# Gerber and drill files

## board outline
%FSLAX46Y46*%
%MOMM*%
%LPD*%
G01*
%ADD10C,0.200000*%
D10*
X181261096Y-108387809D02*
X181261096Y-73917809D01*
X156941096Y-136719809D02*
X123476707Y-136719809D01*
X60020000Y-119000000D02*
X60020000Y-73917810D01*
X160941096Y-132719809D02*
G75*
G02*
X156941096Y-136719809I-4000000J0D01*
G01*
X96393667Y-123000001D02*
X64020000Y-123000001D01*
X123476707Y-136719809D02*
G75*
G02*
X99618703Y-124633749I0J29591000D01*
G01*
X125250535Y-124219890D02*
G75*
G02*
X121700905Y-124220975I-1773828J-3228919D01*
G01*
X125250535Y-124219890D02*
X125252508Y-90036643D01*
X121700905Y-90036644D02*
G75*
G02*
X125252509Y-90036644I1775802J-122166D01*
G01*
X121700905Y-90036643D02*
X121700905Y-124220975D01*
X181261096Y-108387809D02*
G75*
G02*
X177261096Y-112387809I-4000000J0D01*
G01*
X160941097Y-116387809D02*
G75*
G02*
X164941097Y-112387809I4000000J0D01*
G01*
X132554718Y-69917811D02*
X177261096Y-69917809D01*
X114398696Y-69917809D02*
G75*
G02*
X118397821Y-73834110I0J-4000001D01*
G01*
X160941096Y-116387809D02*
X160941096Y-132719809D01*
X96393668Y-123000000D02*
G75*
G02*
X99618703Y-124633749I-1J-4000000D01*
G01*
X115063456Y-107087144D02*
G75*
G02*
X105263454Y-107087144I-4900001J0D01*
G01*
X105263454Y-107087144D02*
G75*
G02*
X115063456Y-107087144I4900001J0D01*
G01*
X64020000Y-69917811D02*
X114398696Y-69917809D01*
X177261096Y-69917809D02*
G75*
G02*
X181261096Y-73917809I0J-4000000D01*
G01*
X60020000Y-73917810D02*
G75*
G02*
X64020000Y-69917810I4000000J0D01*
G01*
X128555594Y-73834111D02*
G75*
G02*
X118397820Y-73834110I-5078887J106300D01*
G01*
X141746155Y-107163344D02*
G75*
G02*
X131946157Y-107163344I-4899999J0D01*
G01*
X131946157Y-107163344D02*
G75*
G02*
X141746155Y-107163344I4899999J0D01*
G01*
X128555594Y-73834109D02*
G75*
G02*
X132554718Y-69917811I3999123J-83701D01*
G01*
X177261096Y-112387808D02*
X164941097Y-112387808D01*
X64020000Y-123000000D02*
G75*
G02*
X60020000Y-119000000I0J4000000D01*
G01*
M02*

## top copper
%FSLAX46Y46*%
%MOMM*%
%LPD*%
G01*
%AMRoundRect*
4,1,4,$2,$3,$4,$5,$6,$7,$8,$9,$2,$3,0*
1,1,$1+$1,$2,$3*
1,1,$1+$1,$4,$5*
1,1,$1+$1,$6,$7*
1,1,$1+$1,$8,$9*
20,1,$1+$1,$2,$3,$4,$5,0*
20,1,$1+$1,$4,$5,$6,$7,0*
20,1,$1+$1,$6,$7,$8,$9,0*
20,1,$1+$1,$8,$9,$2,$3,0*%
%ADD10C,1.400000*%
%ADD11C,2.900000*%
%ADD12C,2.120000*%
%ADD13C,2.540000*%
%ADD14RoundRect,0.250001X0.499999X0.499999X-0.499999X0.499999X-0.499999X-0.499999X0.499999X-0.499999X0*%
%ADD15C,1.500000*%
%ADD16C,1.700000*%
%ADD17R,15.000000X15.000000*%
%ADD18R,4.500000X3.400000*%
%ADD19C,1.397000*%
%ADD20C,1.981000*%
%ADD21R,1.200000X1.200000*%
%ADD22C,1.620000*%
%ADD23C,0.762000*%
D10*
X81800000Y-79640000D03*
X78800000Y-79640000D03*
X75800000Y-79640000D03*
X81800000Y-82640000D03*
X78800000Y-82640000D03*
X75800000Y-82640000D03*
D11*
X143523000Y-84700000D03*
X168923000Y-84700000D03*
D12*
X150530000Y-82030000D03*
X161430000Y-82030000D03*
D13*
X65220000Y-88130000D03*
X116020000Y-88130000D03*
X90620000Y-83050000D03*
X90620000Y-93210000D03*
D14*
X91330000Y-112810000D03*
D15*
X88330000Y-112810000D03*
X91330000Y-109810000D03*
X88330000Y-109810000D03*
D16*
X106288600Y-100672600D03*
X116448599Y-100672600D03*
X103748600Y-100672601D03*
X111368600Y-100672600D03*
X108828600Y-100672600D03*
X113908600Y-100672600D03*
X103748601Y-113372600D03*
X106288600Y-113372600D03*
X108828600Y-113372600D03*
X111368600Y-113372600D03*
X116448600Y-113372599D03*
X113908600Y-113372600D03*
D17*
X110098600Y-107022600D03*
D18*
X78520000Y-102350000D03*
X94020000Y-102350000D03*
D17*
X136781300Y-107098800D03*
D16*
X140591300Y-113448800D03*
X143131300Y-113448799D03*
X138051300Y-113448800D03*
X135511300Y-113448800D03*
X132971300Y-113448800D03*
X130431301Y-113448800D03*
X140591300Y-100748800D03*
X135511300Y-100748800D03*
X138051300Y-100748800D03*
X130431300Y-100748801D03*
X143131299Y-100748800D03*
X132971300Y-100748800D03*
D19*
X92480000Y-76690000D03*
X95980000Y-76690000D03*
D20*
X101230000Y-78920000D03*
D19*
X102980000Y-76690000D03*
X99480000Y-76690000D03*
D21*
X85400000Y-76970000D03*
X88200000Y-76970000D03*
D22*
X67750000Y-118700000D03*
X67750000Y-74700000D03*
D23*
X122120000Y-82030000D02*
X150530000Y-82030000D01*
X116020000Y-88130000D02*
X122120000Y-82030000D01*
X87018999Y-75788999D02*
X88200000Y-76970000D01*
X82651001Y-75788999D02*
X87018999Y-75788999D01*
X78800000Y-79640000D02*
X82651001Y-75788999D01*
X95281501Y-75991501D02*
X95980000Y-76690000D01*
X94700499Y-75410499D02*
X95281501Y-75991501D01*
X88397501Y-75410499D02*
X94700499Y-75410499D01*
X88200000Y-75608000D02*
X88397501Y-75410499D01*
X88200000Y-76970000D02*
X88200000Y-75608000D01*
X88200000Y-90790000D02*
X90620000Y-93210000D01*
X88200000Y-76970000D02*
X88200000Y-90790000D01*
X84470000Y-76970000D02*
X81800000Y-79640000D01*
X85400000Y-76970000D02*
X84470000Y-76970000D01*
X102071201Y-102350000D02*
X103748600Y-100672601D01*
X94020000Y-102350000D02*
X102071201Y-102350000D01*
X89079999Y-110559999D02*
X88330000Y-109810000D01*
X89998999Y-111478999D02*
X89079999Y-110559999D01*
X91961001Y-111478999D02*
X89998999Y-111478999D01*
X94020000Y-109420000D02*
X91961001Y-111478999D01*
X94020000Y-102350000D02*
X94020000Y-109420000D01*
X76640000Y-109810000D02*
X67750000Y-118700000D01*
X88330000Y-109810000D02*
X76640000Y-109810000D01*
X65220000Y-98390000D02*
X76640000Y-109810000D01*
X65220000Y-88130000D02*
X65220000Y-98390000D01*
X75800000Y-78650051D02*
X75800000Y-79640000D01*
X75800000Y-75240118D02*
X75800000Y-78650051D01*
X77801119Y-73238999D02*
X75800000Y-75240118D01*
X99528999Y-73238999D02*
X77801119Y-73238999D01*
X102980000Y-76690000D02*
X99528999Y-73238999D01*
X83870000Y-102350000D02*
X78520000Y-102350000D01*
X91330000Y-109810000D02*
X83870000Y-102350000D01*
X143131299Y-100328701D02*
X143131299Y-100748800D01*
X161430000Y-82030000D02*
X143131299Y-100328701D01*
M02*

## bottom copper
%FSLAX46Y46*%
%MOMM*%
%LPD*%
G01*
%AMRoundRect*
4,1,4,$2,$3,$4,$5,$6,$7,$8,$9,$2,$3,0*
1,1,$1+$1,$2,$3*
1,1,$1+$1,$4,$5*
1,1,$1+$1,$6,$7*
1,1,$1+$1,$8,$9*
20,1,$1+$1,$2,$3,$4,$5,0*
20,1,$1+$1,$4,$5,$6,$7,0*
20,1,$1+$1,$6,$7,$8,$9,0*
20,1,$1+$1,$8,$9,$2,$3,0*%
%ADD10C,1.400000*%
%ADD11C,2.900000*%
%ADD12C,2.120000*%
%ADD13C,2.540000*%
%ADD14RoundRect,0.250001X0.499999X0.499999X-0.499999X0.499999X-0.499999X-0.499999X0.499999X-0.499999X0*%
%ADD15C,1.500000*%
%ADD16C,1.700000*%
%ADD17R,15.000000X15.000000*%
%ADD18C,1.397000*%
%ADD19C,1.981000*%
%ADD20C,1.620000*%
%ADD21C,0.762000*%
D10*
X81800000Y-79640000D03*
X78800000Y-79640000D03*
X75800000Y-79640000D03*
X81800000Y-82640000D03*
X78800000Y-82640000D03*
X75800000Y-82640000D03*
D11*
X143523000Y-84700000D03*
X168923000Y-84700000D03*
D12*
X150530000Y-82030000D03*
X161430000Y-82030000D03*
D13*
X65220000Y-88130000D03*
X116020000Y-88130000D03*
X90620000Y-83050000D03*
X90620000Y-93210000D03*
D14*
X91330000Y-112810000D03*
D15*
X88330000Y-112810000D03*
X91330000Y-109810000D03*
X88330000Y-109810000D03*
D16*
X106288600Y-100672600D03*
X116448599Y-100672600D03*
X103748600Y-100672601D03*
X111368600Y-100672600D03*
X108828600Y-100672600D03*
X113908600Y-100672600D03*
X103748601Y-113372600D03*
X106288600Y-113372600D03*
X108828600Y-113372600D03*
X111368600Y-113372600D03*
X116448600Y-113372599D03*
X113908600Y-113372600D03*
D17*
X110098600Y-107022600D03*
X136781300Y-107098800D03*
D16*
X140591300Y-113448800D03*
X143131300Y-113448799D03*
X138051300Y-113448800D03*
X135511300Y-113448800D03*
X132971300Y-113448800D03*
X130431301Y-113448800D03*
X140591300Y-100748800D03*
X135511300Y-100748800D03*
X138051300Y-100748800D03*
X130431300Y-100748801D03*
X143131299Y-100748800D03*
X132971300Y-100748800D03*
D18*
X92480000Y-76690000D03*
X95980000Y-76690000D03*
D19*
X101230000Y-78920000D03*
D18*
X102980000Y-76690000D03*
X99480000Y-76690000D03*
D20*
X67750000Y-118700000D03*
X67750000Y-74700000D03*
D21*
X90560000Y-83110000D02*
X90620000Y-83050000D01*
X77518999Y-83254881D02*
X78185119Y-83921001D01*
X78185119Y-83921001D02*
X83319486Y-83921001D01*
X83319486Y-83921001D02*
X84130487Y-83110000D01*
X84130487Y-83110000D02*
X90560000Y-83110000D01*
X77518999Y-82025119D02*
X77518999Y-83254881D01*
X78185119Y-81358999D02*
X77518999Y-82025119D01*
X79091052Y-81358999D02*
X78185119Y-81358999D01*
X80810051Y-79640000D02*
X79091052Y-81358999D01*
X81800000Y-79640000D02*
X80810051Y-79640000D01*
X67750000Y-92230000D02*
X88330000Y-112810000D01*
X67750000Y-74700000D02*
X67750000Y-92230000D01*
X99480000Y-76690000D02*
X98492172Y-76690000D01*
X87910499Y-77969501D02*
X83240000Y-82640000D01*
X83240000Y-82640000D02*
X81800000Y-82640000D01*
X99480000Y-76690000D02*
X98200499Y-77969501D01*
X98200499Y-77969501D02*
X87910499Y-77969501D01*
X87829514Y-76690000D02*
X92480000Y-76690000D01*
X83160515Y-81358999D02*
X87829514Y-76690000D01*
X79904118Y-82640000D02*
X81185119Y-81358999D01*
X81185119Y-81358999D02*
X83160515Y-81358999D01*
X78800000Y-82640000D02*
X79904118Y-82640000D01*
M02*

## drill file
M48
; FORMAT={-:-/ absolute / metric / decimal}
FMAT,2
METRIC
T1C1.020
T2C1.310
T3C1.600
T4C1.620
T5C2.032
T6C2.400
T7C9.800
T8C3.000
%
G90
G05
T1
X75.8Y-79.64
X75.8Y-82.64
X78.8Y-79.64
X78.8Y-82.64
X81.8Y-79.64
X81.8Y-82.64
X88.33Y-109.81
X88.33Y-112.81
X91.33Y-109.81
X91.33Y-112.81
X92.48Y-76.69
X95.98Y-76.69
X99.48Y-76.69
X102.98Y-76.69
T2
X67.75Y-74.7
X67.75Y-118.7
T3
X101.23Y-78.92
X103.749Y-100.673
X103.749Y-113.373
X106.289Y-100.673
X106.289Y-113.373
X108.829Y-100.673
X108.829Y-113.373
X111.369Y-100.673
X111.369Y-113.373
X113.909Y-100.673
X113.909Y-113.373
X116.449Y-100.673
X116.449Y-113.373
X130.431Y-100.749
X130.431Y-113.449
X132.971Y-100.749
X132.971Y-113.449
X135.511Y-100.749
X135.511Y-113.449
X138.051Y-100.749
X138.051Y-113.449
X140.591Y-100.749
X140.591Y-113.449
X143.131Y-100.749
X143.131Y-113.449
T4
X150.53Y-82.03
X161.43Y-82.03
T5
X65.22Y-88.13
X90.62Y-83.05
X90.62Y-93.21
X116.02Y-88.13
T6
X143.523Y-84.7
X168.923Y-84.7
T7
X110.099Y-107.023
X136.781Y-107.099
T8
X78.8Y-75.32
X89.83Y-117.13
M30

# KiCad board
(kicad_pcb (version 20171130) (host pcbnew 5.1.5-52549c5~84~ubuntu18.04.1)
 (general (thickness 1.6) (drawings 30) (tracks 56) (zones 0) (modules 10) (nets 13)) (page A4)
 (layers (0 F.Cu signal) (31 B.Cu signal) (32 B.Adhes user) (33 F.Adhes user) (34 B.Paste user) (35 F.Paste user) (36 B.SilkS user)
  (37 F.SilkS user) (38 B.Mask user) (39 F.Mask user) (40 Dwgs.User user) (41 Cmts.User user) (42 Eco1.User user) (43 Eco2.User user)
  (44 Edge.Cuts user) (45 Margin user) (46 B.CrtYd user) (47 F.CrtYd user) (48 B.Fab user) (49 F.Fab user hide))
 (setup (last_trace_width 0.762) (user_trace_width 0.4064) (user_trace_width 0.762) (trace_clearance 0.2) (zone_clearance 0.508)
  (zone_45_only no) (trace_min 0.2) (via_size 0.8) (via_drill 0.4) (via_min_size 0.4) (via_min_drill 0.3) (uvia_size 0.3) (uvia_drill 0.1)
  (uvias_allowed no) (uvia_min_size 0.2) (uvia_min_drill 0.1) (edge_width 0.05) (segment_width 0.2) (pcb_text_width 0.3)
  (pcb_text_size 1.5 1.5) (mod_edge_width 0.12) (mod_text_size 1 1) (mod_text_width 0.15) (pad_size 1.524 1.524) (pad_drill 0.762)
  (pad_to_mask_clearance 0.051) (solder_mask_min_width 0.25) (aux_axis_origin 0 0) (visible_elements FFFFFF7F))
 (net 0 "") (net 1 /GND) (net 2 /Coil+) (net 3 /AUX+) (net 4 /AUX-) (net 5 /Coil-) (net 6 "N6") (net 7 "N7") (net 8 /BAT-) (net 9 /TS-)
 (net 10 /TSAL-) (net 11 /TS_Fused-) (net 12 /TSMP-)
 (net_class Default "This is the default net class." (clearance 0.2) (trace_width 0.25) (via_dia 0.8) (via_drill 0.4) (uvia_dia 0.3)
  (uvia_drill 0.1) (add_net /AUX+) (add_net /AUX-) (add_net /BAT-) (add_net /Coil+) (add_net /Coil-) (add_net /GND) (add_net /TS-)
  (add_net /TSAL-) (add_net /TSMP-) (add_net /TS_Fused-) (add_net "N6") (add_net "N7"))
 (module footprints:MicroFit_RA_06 (layer B.Cu) (at 78.8 75.32 180)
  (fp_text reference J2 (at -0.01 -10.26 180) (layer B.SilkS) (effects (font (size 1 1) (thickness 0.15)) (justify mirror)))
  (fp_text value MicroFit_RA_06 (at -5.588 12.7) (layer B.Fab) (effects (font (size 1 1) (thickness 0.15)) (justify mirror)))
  (pad "" np_thru_hole circle (at 0 0) (size 3 3) (drill 3) (layers *.Cu *.Mask))
  (pad 1 thru_hole circle (at -3 -4.32) (size 1.4 1.4) (drill 1.02) (layers *.Cu *.Mask) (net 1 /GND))
  (pad 2 thru_hole circle (at 0 -4.32) (size 1.4 1.4) (drill 1.02) (layers *.Cu *.Mask) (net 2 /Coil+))
  (pad 3 thru_hole circle (at 3 -4.32) (size 1.4 1.4) (drill 1.02) (layers *.Cu *.Mask) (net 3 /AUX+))
  (pad 4 thru_hole circle (at -3 -7.32) (size 1.4 1.4) (drill 1.02) (layers *.Cu *.Mask) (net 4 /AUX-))
  (pad 5 thru_hole circle (at 0 -7.32) (size 1.4 1.4) (drill 1.02) (layers *.Cu *.Mask) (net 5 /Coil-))
  (pad 6 thru_hole circle (at 3 -7.32) (size 1.4 1.4) (drill 1.02) (layers *.Cu *.Mask) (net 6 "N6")))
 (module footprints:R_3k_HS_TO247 (layer F.Cu) (at 161.43 82.03 180)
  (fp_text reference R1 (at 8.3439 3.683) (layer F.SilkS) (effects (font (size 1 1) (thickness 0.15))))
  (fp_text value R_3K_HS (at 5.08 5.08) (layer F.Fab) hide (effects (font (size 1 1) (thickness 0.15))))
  (pad 5 thru_hole circle (at 17.907 -2.67 180) (size 2.9 2.9) (drill 2.4) (layers *.Cu *.Mask))
  (pad 4 thru_hole circle (at -7.493 -2.67 180) (size 2.9 2.9) (drill 2.4) (layers *.Cu *.Mask))
  (pad 2 thru_hole circle (at 10.9 0 180) (size 2.12 2.12) (drill 1.62) (layers *.Cu *.Mask) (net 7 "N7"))
  (pad 1 thru_hole circle (at 0 0 180) (size 2.12 2.12) (drill 1.62) (layers *.Cu *.Mask) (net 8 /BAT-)))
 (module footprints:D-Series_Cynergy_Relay (layer F.Cu) (at 65.22 88.13)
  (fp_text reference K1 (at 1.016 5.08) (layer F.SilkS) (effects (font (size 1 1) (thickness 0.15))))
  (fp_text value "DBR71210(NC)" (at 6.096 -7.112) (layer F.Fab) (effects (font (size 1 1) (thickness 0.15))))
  (pad 1 thru_hole circle (at 0 0) (size 2.54 2.54) (drill 2.032) (layers *.Cu *.Mask) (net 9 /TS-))
  (pad 2 thru_hole circle (at 50.8 0) (size 2.54 2.54) (drill 2.032) (layers *.Cu *.Mask) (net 7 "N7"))
  (pad 3 thru_hole circle (at 25.4 -5.08) (size 2.54 2.54) (drill 2.032) (layers *.Cu *.Mask) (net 1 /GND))
  (pad 4 thru_hole circle (at 25.4 5.08) (size 2.54 2.54) (drill 2.032) (layers *.Cu *.Mask) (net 2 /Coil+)))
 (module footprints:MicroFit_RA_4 (layer F.Cu) (at 91.33 112.81 180)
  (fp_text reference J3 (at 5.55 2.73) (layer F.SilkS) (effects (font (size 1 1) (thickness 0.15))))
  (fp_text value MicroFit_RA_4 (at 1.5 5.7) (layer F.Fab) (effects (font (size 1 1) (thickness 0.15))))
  (pad "" np_thru_hole circle (at 1.5 -4.32 180) (size 3 3) (drill 3) (layers *.Cu *.Mask))
  (pad 1 thru_hole roundrect (at 0 0 180) (size 1.5 1.5) (drill 1.02) (layers *.Cu *.Mask) (roundrect_rratio 0.166667) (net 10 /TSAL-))
  (pad 2 thru_hole circle (at 3 0 180) (size 1.5 1.5) (drill 1.02) (layers *.Cu *.Mask) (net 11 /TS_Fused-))
  (pad 3 thru_hole circle (at 0 3 180) (size 1.5 1.5) (drill 1.02) (layers *.Cu *.Mask) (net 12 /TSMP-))
  (pad 4 thru_hole circle (at 3 3 180) (size 1.5 1.5) (drill 1.02) (layers *.Cu *.Mask) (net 9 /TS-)))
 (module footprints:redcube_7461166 (layer F.Cu) (at 110.0986 107.0226)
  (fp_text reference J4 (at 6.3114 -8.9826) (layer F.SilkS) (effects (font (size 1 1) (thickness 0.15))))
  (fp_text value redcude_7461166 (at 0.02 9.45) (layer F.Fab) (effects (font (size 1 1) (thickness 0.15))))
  (pad 1 thru_hole circle (at -3.81 -6.35) (size 1.7 1.7) (drill 1.6) (layers *.Cu *.Mask) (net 9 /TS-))
  (pad 1 thru_hole circle (at 6.349999 -6.35) (size 1.7 1.7) (drill 1.6) (layers *.Cu *.Mask) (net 9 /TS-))
  (pad 1 thru_hole circle (at -6.35 -6.349999) (size 1.7 1.7) (drill 1.6) (layers *.Cu *.Mask) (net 9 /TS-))
  (pad 1 thru_hole circle (at 1.27 -6.35) (size 1.7 1.7) (drill 1.6) (layers *.Cu *.Mask) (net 9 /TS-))
  (pad 1 thru_hole circle (at -1.27 -6.35) (size 1.7 1.7) (drill 1.6) (layers *.Cu *.Mask) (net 9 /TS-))
  (pad 1 thru_hole circle (at 3.81 -6.35) (size 1.7 1.7) (drill 1.6) (layers *.Cu *.Mask) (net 9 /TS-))
  (pad 1 thru_hole circle (at -6.349999 6.35) (size 1.7 1.7) (drill 1.6) (layers *.Cu *.Mask) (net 9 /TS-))
  (pad 1 thru_hole circle (at -3.81 6.35) (size 1.7 1.7) (drill 1.6) (layers *.Cu *.Mask) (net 9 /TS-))
  (pad 1 thru_hole circle (at -1.27 6.35) (size 1.7 1.7) (drill 1.6) (layers *.Cu *.Mask) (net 9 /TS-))
  (pad 1 thru_hole circle (at 1.27 6.35) (size 1.7 1.7) (drill 1.6) (layers *.Cu *.Mask) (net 9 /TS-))
  (pad 1 thru_hole circle (at 6.35 6.349999) (size 1.7 1.7) (drill 1.6) (layers *.Cu *.Mask) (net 9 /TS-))
  (pad 1 thru_hole circle (at 3.81 6.35) (size 1.7 1.7) (drill 1.6) (layers *.Cu *.Mask) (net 9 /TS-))
  (pad 1 thru_hole rect (at 0 0) (size 15 15) (drill 9.8) (layers *.Cu *.Mask) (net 9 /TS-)))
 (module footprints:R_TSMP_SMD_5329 (layer F.Cu) (at 86.14 102.35)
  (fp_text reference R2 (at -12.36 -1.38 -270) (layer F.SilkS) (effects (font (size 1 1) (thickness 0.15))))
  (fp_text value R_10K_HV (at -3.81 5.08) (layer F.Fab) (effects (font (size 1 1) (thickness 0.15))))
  (pad 1 smd rect (at -7.62 0) (size 4.5 3.4) (layers F.Cu F.Paste F.Mask) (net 12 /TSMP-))
  (pad 2 smd rect (at 7.88 0) (size 4.5 3.4) (layers F.Cu F.Paste F.Mask) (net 9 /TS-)))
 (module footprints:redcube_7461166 (layer F.Cu) (at 136.7813 107.0988)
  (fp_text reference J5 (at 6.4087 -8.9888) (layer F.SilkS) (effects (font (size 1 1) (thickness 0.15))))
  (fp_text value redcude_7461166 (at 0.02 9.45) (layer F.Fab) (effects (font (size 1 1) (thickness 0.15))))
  (pad 1 thru_hole rect (at 0 0) (size 15 15) (drill 9.8) (layers *.Cu *.Mask) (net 8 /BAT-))
  (pad 1 thru_hole circle (at 3.81 6.35) (size 1.7 1.7) (drill 1.6) (layers *.Cu *.Mask) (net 8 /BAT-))
  (pad 1 thru_hole circle (at 6.35 6.349999) (size 1.7 1.7) (drill 1.6) (layers *.Cu *.Mask) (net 8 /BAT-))
  (pad 1 thru_hole circle (at 1.27 6.35) (size 1.7 1.7) (drill 1.6) (layers *.Cu *.Mask) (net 8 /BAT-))
  (pad 1 thru_hole circle (at -1.27 6.35) (size 1.7 1.7) (drill 1.6) (layers *.Cu *.Mask) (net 8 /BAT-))
  (pad 1 thru_hole circle (at -3.81 6.35) (size 1.7 1.7) (drill 1.6) (layers *.Cu *.Mask) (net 8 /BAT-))
  (pad 1 thru_hole circle (at -6.349999 6.35) (size 1.7 1.7) (drill 1.6) (layers *.Cu *.Mask) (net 8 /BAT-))
  (pad 1 thru_hole circle (at 3.81 -6.35) (size 1.7 1.7) (drill 1.6) (layers *.Cu *.Mask) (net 8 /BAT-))
  (pad 1 thru_hole circle (at -1.27 -6.35) (size 1.7 1.7) (drill 1.6) (layers *.Cu *.Mask) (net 8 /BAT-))
  (pad 1 thru_hole circle (at 1.27 -6.35) (size 1.7 1.7) (drill 1.6) (layers *.Cu *.Mask) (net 8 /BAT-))
  (pad 1 thru_hole circle (at -6.35 -6.349999) (size 1.7 1.7) (drill 1.6) (layers *.Cu *.Mask) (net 8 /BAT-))
  (pad 1 thru_hole circle (at 6.349999 -6.35) (size 1.7 1.7) (drill 1.6) (layers *.Cu *.Mask) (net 8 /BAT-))
  (pad 1 thru_hole circle (at -3.81 -6.35) (size 1.7 1.7) (drill 1.6) (layers *.Cu *.Mask) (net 8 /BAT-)))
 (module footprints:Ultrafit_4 (layer B.Cu) (at 97.73 76.69 270)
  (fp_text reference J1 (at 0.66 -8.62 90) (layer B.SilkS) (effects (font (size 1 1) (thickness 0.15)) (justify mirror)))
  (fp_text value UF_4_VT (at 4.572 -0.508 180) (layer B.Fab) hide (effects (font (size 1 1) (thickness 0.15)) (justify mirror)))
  (pad 4 thru_hole circle (at 0 5.25 90) (size 1.397 1.397) (drill 1.02) (layers *.Cu *.Mask) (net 5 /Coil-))
  (pad 3 thru_hole circle (at 0 1.75 90) (size 1.397 1.397) (drill 1.02) (layers *.Cu *.Mask) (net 2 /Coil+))
  (pad "" thru_hole circle (at 2.23 -3.5 270) (size 1.981 1.981) (drill 1.6) (layers *.Cu *.Mask))
  (pad 1 thru_hole circle (at 0 -5.25 270) (size 1.397 1.397) (drill 1.02) (layers *.Cu *.Mask) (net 3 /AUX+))
  (pad 2 thru_hole circle (at 0 -1.75 270) (size 1.397 1.397) (drill 1.02) (layers *.Cu *.Mask) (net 4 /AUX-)))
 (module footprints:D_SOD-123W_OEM (layer F.Cu) (at 86.8 76.97 180)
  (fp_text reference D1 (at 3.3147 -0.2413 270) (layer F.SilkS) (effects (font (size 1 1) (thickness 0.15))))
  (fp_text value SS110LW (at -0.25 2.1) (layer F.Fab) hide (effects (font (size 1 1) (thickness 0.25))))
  (pad 2 smd rect (at 1.4 0 180) (size 1.2 1.2) (layers F.Cu F.Paste F.Mask) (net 1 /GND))
  (pad 1 smd rect (at -1.4 0 180) (size 1.2 1.2) (layers F.Cu F.Paste F.Mask) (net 2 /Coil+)))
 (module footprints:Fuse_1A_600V (layer B.Cu) (at 67.75 118.7 90)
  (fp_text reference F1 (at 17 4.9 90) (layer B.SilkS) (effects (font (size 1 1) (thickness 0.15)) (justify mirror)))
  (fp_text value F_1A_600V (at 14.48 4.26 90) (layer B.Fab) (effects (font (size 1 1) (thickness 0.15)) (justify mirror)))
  (pad 1 thru_hole circle (at 0 0 90) (size 1.62 1.62) (drill 1.31) (layers *.Cu *.Mask) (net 9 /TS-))
  (pad 2 thru_hole circle (at 44 0 90) (size 1.62 1.62) (drill 1.31) (layers *.Cu *.Mask) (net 11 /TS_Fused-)))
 (gr_line (start 181.261096 108.387809) (end 181.261096 73.917809) (layer Edge.Cuts) (width 0.2))
 (gr_line (start 156.941096 136.719809) (end 123.476707 136.719809) (layer Edge.Cuts) (width 0.2))
 (gr_line (start 60.02 119) (end 60.02 73.91781) (layer Edge.Cuts) (width 0.2))
 (gr_arc (start 156.941096 132.719809) (end 156.941096 136.719809) (angle -90) (layer Edge.Cuts) (width 0.2))
 (gr_line (start 96.393667 123.000001) (end 64.02 123.000001) (layer Edge.Cuts) (width 0.2))
 (gr_arc (start 123.476707 107.128809) (end 99.618703 124.633749) (angle -53.73199979) (layer Edge.Cuts) (width 0.2))
 (gr_arc (start 123.476707 127.448809) (end 121.700905 124.220975) (angle -302.4) (layer Edge.Cuts) (width 0.2))
 (gr_line (start 125.250535 124.21989) (end 125.252508 90.036643) (layer Edge.Cuts) (width 0.2))
 (gr_arc (start 123.476707 90.15881) (end 125.252509 90.036644) (angle -172.1290943) (layer Edge.Cuts) (width 0.2))
 (gr_line (start 121.700905 90.036643) (end 121.700905 124.220975) (layer Edge.Cuts) (width 0.2))
 (gr_arc (start 177.261096 108.387809) (end 177.261096 112.387809) (angle -90) (layer Edge.Cuts) (width 0.2))
 (gr_arc (start 164.941097 116.387809) (end 164.941097 112.387809) (angle -90) (layer Edge.Cuts) (width 0.2))
 (gr_line (start 132.554718 69.917811) (end 177.261096 69.917809) (layer Edge.Cuts) (width 0.2))
 (gr_arc (start 114.398696 73.91781) (end 118.397821 73.83411) (angle -88.80099199) (layer Edge.Cuts) (width 0.2))
 (gr_line (start 160.941096 116.387809) (end 160.941096 132.719809) (layer Edge.Cuts) (width 0.2))
 (gr_arc (start 96.393667 127) (end 99.618703 124.633749) (angle -53.73200771) (layer Edge.Cuts) (width 0.2))
 (gr_circle (center 110.163455 107.087144) (end 115.063456 107.087144) (layer Edge.Cuts) (width 0.2))
 (gr_line (start 64.02 69.917811) (end 114.398696 69.917809) (layer Edge.Cuts) (width 0.2))
 (gr_arc (start 177.261096 73.917809) (end 181.261096 73.917809) (angle -90.00000194) (layer Edge.Cuts) (width 0.2))
 (gr_arc (start 64.02 73.91781) (end 64.02 69.91781) (angle -90) (layer Edge.Cuts) (width 0.2))
 (gr_arc (start 123.476707 73.727811) (end 118.39782 73.83411) (angle -177.6019899) (layer Edge.Cuts) (width 0.2))
 (gr_circle (center 136.846156 107.163344) (end 141.746155 107.163344) (layer Edge.Cuts) (width 0.2))
 (gr_arc (start 132.554717 73.91781) (end 132.554718 69.917811) (angle -88.80099199) (layer Edge.Cuts) (width 0.2))
 (gr_line (start 177.261096 112.387808) (end 164.941097 112.387808) (layer Edge.Cuts) (width 0.2))
 (gr_arc (start 64.02 119) (end 60.02 119) (angle -90) (layer Edge.Cuts) (width 0.2))
 (segment (start 122.12 82.03) (end 150.53 82.03) (width 0.762) (layer F.Cu) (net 7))
 (segment (start 116.02 88.13) (end 122.12 82.03) (width 0.762) (layer F.Cu) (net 7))
 (segment (start 87.018999 75.788999) (end 88.2 76.97) (width 0.762) (layer F.Cu) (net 2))
 (segment (start 82.651001 75.788999) (end 87.018999 75.788999) (width 0.762) (layer F.Cu) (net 2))
 (segment (start 78.8 79.64) (end 82.651001 75.788999) (width 0.762) (layer F.Cu) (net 2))
 (segment (start 95.281501 75.991501) (end 95.98 76.69) (width 0.762) (layer F.Cu) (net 2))
 (segment (start 94.700499 75.410499) (end 95.281501 75.991501) (width 0.762) (layer F.Cu) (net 2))
 (segment (start 88.397501 75.410499) (end 94.700499 75.410499) (width 0.762) (layer F.Cu) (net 2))
 (segment (start 88.2 75.608) (end 88.397501 75.410499) (width 0.762) (layer F.Cu) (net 2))
 (segment (start 88.2 76.97) (end 88.2 75.608) (width 0.762) (layer F.Cu) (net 2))
 (segment (start 88.2 90.79) (end 90.62 93.21) (width 0.762) (layer F.Cu) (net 2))
 (segment (start 88.2 76.97) (end 88.2 90.79) (width 0.762) (layer F.Cu) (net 2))
 (segment (start 84.47 76.97) (end 81.8 79.64) (width 0.762) (layer F.Cu) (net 1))
 (segment (start 85.4 76.97) (end 84.47 76.97) (width 0.762) (layer F.Cu) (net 1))
 (segment (start 90.56 83.11) (end 90.62 83.05) (width 0.762) (layer B.Cu) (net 1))
 (segment (start 77.518999 83.254881) (end 78.185119 83.921001) (width 0.762) (layer B.Cu) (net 1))
 (segment (start 78.185119 83.921001) (end 83.319486 83.921001) (width 0.762) (layer B.Cu) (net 1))
 (segment (start 83.319486 83.921001) (end 84.130487 83.11) (width 0.762) (layer B.Cu) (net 1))
 (segment (start 84.130487 83.11) (end 90.56 83.11) (width 0.762) (layer B.Cu) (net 1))
 (segment (start 77.518999 82.025119) (end 77.518999 83.254881) (width 0.762) (layer B.Cu) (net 1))
 (segment (start 78.185119 81.358999) (end 77.518999 82.025119) (width 0.762) (layer B.Cu) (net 1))
 (segment (start 79.091052 81.358999) (end 78.185119 81.358999) (width 0.762) (layer B.Cu) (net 1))
 (segment (start 80.810051 79.64) (end 79.091052 81.358999) (width 0.762) (layer B.Cu) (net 1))
 (segment (start 81.8 79.64) (end 80.810051 79.64) (width 0.762) (layer B.Cu) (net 1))
 (segment (start 67.75 92.23) (end 88.33 112.81) (width 0.762) (layer B.Cu) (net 11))
 (segment (start 67.75 74.7) (end 67.75 92.23) (width 0.762) (layer B.Cu) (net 11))
 (segment (start 102.071201 102.35) (end 103.7486 100.672601) (width 0.762) (layer F.Cu) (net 9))
 (segment (start 94.02 102.35) (end 102.071201 102.35) (width 0.762) (layer F.Cu) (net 9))
 (segment (start 89.079999 110.559999) (end 88.33 109.81) (width 0.762) (layer F.Cu) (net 9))
 (segment (start 89.998999 111.478999) (end 89.079999 110.559999) (width 0.762) (layer F.Cu) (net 9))
 (segment (start 91.961001 111.478999) (end 89.998999 111.478999) (width 0.762) (layer F.Cu) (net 9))
 (segment (start 94.02 109.42) (end 91.961001 111.478999) (width 0.762) (layer F.Cu) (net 9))
 (segment (start 94.02 102.35) (end 94.02 109.42) (width 0.762) (layer F.Cu) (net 9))
 (segment (start 76.64 109.81) (end 67.75 118.7) (width 0.762) (layer F.Cu) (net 9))
 (segment (start 88.33 109.81) (end 76.64 109.81) (width 0.762) (layer F.Cu) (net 9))
 (segment (start 65.22 98.39) (end 76.64 109.81) (width 0.762) (layer F.Cu) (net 9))
 (segment (start 65.22 88.13) (end 65.22 98.39) (width 0.762) (layer F.Cu) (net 9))
 (segment (start 99.48 76.69) (end 98.492172 76.69) (width 0.762) (layer B.Cu) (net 4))
 (segment (start 87.910499 77.969501) (end 83.24 82.64) (width 0.762) (layer B.Cu) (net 4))
 (segment (start 83.24 82.64) (end 81.8 82.64) (width 0.762) (layer B.Cu) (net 4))
 (segment (start 99.48 76.69) (end 98.200499 77.969501) (width 0.762) (layer B.Cu) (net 4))
 (segment (start 98.200499 77.969501) (end 87.910499 77.969501) (width 0.762) (layer B.Cu) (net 4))
 (segment (start 87.829514 76.69) (end 92.48 76.69) (width 0.762) (layer B.Cu) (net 5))
 (segment (start 83.160515 81.358999) (end 87.829514 76.69) (width 0.762) (layer B.Cu) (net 5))
 (segment (start 79.904118 82.64) (end 81.185119 81.358999) (width 0.762) (layer B.Cu) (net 5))
 (segment (start 81.185119 81.358999) (end 83.160515 81.358999) (width 0.762) (layer B.Cu) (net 5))
 (segment (start 78.8 82.64) (end 79.904118 82.64) (width 0.762) (layer B.Cu) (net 5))
 (segment (start 75.8 78.650051) (end 75.8 79.64) (width 0.762) (layer F.Cu) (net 3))
 (segment (start 75.8 75.240118) (end 75.8 78.650051) (width 0.762) (layer F.Cu) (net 3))
 (segment (start 77.801119 73.238999) (end 75.8 75.240118) (width 0.762) (layer F.Cu) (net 3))
 (segment (start 99.528999 73.238999) (end 77.801119 73.238999) (width 0.762) (layer F.Cu) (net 3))
 (segment (start 102.98 76.69) (end 99.528999 73.238999) (width 0.762) (layer F.Cu) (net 3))
 (segment (start 83.87 102.35) (end 78.52 102.35) (width 0.762) (layer F.Cu) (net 12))
 (segment (start 91.33 109.81) (end 83.87 102.35) (width 0.762) (layer F.Cu) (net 12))
 (segment (start 143.131299 100.328701) (end 143.131299 100.7488) (width 0.762) (layer F.Cu) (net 8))
 (segment (start 161.43 82.03) (end 143.131299 100.328701) (width 0.762) (layer F.Cu) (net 8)))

